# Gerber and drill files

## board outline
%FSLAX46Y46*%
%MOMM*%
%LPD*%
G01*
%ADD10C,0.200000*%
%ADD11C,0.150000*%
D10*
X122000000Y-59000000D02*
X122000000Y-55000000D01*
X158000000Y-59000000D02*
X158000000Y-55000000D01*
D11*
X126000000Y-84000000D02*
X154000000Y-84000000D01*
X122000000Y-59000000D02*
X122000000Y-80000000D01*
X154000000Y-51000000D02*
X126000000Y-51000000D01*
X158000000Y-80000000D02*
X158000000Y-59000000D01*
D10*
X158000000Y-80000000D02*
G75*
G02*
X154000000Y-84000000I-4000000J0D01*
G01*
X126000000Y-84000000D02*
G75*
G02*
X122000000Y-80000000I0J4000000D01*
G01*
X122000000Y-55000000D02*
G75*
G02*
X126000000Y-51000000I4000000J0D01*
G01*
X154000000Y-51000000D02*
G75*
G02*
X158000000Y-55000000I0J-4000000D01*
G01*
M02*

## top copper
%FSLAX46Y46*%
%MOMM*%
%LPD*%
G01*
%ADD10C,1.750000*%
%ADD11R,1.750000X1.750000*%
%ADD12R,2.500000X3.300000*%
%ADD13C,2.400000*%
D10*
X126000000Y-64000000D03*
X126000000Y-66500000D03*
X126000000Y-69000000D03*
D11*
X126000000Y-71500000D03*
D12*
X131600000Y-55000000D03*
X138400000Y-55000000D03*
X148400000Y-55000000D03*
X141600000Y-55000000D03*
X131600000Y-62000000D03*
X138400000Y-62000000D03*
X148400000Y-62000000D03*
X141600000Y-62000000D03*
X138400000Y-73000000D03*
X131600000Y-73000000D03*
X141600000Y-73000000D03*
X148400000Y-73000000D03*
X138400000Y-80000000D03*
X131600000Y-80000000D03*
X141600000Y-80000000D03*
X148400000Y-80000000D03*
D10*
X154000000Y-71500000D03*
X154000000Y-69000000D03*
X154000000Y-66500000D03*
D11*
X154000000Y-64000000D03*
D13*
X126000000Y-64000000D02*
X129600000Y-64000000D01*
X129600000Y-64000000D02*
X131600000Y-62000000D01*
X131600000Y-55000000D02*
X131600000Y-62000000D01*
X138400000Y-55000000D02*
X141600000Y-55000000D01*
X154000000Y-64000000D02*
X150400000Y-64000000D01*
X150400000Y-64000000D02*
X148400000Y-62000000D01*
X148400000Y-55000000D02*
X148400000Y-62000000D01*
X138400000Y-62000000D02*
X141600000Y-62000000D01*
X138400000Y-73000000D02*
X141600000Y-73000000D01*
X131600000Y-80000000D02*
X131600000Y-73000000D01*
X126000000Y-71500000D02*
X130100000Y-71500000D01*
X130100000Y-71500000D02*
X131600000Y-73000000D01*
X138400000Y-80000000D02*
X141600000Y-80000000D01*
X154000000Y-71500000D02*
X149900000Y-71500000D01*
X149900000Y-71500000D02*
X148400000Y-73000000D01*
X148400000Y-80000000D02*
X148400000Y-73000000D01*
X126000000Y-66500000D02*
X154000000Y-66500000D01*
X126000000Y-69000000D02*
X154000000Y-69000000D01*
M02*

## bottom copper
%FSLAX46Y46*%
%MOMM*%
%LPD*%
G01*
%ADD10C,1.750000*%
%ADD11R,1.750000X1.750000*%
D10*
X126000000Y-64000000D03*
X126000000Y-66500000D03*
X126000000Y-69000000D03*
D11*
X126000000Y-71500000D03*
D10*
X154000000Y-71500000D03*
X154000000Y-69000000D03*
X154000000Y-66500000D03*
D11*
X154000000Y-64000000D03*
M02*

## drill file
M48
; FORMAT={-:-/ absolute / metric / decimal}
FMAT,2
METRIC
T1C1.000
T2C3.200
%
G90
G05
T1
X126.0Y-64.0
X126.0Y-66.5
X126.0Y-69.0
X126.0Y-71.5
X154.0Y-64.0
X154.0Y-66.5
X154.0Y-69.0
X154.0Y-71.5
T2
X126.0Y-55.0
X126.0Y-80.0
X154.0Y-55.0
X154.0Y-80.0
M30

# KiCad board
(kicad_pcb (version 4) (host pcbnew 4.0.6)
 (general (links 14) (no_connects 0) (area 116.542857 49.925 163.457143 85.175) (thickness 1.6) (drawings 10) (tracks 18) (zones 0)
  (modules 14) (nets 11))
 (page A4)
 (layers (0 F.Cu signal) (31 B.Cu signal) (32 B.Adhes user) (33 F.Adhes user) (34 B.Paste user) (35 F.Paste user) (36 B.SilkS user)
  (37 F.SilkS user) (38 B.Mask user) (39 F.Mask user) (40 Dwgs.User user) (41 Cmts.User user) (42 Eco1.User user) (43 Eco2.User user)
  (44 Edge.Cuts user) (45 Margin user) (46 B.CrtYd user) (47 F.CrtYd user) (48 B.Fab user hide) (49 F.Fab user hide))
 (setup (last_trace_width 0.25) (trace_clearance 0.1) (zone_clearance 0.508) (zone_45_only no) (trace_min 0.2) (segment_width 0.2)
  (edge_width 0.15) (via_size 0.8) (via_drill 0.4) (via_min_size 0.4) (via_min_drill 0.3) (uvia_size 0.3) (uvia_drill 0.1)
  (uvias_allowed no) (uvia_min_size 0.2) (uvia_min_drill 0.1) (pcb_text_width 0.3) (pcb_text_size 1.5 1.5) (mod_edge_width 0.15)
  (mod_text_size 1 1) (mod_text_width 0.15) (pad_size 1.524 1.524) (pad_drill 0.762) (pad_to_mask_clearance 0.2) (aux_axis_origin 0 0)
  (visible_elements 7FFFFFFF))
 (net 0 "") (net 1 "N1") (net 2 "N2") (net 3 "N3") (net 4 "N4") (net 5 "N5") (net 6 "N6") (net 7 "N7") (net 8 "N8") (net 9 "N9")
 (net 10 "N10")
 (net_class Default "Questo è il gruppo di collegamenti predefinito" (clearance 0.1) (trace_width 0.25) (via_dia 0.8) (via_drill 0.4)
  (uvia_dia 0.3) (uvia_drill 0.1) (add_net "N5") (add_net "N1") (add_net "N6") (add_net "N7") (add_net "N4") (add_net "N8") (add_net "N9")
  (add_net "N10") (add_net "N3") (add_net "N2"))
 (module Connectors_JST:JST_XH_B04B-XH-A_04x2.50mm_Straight (layer F.Cu) (at 126 71.5 90)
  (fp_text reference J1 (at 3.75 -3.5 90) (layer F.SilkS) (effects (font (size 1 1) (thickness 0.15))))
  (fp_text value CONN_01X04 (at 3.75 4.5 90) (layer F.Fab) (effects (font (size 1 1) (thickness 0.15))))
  (pad 4 thru_hole circle (at 7.5 0 90) (size 1.75 1.75) (drill 1) (layers *.Cu *.Mask) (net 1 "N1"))
  (pad 3 thru_hole circle (at 5 0 90) (size 1.75 1.75) (drill 1) (layers *.Cu *.Mask) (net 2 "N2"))
  (pad 2 thru_hole circle (at 2.5 0 90) (size 1.75 1.75) (drill 1) (layers *.Cu *.Mask) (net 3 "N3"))
  (pad 1 thru_hole rect (at 0 0 90) (size 1.75 1.75) (drill 1) (layers *.Cu *.Mask) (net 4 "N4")))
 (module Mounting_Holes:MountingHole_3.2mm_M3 (layer F.Cu) (at 126 55)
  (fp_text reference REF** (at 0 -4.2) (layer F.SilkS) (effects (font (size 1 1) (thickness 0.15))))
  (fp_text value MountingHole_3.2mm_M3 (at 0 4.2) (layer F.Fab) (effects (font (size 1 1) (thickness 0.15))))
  (pad 1 np_thru_hole circle (at 0 0) (size 3.2 3.2) (drill 3.2) (layers *.Cu *.Mask)))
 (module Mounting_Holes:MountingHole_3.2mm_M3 (layer F.Cu) (at 154 55)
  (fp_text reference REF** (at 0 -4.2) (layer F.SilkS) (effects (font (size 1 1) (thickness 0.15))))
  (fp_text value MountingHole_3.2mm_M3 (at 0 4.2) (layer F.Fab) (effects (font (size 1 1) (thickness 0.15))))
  (pad 1 np_thru_hole circle (at 0 0) (size 3.2 3.2) (drill 3.2) (layers *.Cu *.Mask)))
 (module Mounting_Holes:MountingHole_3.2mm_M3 (layer F.Cu) (at 154 80)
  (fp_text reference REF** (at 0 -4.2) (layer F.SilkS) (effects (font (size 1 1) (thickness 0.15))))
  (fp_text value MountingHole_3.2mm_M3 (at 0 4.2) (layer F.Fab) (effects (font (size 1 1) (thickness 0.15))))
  (pad 1 np_thru_hole circle (at 0 0) (size 3.2 3.2) (drill 3.2) (layers *.Cu *.Mask)))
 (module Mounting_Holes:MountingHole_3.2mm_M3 (layer F.Cu) (at 126 80)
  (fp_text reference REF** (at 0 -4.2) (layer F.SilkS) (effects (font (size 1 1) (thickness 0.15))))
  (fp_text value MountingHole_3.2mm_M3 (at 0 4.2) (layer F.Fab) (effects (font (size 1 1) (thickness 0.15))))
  (pad 1 np_thru_hole circle (at 0 0) (size 3.2 3.2) (drill 3.2) (layers *.Cu *.Mask)))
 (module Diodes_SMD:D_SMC (layer F.Cu) (at 135 55 180)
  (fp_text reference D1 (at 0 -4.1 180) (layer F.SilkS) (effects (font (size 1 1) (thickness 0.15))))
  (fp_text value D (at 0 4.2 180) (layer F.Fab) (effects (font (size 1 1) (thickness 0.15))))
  (pad 2 smd rect (at 3.4 0 270) (size 3.3 2.5) (layers F.Cu F.Paste F.Mask) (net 1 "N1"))
  (pad 1 smd rect (at -3.4 0 270) (size 3.3 2.5) (layers F.Cu F.Paste F.Mask) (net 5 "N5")))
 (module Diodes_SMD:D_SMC (layer F.Cu) (at 145 55 180)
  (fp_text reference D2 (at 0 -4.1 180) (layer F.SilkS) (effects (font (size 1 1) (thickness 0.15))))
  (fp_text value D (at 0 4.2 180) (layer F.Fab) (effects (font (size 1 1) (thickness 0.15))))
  (pad 1 smd rect (at -3.4 0 270) (size 3.3 2.5) (layers F.Cu F.Paste F.Mask) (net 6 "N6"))
  (pad 2 smd rect (at 3.4 0 270) (size 3.3 2.5) (layers F.Cu F.Paste F.Mask) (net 5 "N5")))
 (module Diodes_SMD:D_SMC (layer F.Cu) (at 135 62)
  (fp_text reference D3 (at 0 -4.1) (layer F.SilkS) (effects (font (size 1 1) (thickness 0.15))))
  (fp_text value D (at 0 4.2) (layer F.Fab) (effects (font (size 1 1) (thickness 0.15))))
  (pad 1 smd rect (at -3.4 0 90) (size 3.3 2.5) (layers F.Cu F.Paste F.Mask) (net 1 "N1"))
  (pad 2 smd rect (at 3.4 0 90) (size 3.3 2.5) (layers F.Cu F.Paste F.Mask) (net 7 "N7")))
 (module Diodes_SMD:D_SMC (layer F.Cu) (at 145 62)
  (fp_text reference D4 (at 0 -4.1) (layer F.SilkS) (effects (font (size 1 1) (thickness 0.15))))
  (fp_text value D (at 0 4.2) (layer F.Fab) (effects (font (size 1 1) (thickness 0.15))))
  (pad 2 smd rect (at 3.4 0 90) (size 3.3 2.5) (layers F.Cu F.Paste F.Mask) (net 6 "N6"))
  (pad 1 smd rect (at -3.4 0 90) (size 3.3 2.5) (layers F.Cu F.Paste F.Mask) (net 7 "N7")))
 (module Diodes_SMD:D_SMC (layer F.Cu) (at 135 73)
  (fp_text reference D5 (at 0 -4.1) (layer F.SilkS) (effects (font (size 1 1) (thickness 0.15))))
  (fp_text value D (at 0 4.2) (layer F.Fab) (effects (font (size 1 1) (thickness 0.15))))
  (pad 2 smd rect (at 3.4 0 90) (size 3.3 2.5) (layers F.Cu F.Paste F.Mask) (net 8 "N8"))
  (pad 1 smd rect (at -3.4 0 90) (size 3.3 2.5) (layers F.Cu F.Paste F.Mask) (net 4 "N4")))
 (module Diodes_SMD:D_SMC (layer F.Cu) (at 145 73)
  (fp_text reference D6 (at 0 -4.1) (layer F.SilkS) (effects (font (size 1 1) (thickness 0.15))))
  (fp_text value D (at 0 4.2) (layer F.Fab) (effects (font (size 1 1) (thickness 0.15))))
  (pad 1 smd rect (at -3.4 0 90) (size 3.3 2.5) (layers F.Cu F.Paste F.Mask) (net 8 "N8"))
  (pad 2 smd rect (at 3.4 0 90) (size 3.3 2.5) (layers F.Cu F.Paste F.Mask) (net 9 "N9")))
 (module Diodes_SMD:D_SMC (layer F.Cu) (at 135 80 180)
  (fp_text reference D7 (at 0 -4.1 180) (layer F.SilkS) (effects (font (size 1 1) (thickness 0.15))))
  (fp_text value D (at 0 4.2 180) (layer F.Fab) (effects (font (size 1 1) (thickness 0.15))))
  (pad 1 smd rect (at -3.4 0 270) (size 3.3 2.5) (layers F.Cu F.Paste F.Mask) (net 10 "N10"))
  (pad 2 smd rect (at 3.4 0 270) (size 3.3 2.5) (layers F.Cu F.Paste F.Mask) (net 4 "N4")))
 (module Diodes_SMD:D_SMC (layer F.Cu) (at 145 80 180)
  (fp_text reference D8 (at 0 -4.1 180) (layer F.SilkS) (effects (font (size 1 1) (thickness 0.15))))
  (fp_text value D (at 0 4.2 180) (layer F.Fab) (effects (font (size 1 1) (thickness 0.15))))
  (pad 2 smd rect (at 3.4 0 270) (size 3.3 2.5) (layers F.Cu F.Paste F.Mask) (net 10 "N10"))
  (pad 1 smd rect (at -3.4 0 270) (size 3.3 2.5) (layers F.Cu F.Paste F.Mask) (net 9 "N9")))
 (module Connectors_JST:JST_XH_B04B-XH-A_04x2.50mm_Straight (layer F.Cu) (at 154 64 270)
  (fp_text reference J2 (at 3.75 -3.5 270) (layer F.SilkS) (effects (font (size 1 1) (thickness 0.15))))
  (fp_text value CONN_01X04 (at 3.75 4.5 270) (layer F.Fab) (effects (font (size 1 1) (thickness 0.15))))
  (pad 4 thru_hole circle (at 7.5 0 270) (size 1.75 1.75) (drill 1) (layers *.Cu *.Mask) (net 9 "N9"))
  (pad 3 thru_hole circle (at 5 0 270) (size 1.75 1.75) (drill 1) (layers *.Cu *.Mask) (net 3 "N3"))
  (pad 2 thru_hole circle (at 2.5 0 270) (size 1.75 1.75) (drill 1) (layers *.Cu *.Mask) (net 2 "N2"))
  (pad 1 thru_hole rect (at 0 0 270) (size 1.75 1.75) (drill 1) (layers *.Cu *.Mask) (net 6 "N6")))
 (gr_line (start 122 59) (end 122 55) (layer Edge.Cuts) (width 0.2))
 (gr_line (start 158 59) (end 158 55) (layer Edge.Cuts) (width 0.2))
 (gr_line (start 126 84) (end 154 84) (layer Edge.Cuts) (width 0.15))
 (gr_line (start 122 59) (end 122 80) (layer Edge.Cuts) (width 0.15))
 (gr_line (start 154 51) (end 126 51) (layer Edge.Cuts) (width 0.15))
 (gr_line (start 158 80) (end 158 59) (layer Edge.Cuts) (width 0.15))
 (gr_arc (start 154 80) (end 154 84) (angle -90) (layer Edge.Cuts) (width 0.2))
 (gr_arc (start 126 80) (end 122 80) (angle -90) (layer Edge.Cuts) (width 0.2))
 (gr_arc (start 126 55) (end 126 51) (angle -90) (layer Edge.Cuts) (width 0.2))
 (gr_arc (start 154 55) (end 158 55) (angle -90) (layer Edge.Cuts) (width 0.2))
 (segment (start 126 64) (end 129.6 64) (width 2.4) (layer F.Cu) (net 1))
 (segment (start 129.6 64) (end 131.6 62) (width 2.4) (layer F.Cu) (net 1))
 (segment (start 131.6 55) (end 131.6 62) (width 2.4) (layer F.Cu) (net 1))
 (segment (start 138.4 55) (end 141.6 55) (width 2.4) (layer F.Cu) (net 5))
 (segment (start 154 64) (end 150.4 64) (width 2.4) (layer F.Cu) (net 6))
 (segment (start 150.4 64) (end 148.4 62) (width 2.4) (layer F.Cu) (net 6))
 (segment (start 148.4 55) (end 148.4 62) (width 2.4) (layer F.Cu) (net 6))
 (segment (start 138.4 62) (end 141.6 62) (width 2.4) (layer F.Cu) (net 7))
 (segment (start 138.4 73) (end 141.6 73) (width 2.4) (layer F.Cu) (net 8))
 (segment (start 131.6 80) (end 131.6 73) (width 2.4) (layer F.Cu) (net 4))
 (segment (start 126 71.5) (end 130.1 71.5) (width 2.4) (layer F.Cu) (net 4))
 (segment (start 130.1 71.5) (end 131.6 73) (width 2.4) (layer F.Cu) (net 4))
 (segment (start 138.4 80) (end 141.6 80) (width 2.4) (layer F.Cu) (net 10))
 (segment (start 154 71.5) (end 149.9 71.5) (width 2.4) (layer F.Cu) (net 9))
 (segment (start 149.9 71.5) (end 148.4 73) (width 2.4) (layer F.Cu) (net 9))
 (segment (start 148.4 80) (end 148.4 73) (width 2.4) (layer F.Cu) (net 9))
 (segment (start 126 66.5) (end 154 66.5) (width 2.4) (layer F.Cu) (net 2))
 (segment (start 126 69) (end 154 69) (width 2.4) (layer F.Cu) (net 3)))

